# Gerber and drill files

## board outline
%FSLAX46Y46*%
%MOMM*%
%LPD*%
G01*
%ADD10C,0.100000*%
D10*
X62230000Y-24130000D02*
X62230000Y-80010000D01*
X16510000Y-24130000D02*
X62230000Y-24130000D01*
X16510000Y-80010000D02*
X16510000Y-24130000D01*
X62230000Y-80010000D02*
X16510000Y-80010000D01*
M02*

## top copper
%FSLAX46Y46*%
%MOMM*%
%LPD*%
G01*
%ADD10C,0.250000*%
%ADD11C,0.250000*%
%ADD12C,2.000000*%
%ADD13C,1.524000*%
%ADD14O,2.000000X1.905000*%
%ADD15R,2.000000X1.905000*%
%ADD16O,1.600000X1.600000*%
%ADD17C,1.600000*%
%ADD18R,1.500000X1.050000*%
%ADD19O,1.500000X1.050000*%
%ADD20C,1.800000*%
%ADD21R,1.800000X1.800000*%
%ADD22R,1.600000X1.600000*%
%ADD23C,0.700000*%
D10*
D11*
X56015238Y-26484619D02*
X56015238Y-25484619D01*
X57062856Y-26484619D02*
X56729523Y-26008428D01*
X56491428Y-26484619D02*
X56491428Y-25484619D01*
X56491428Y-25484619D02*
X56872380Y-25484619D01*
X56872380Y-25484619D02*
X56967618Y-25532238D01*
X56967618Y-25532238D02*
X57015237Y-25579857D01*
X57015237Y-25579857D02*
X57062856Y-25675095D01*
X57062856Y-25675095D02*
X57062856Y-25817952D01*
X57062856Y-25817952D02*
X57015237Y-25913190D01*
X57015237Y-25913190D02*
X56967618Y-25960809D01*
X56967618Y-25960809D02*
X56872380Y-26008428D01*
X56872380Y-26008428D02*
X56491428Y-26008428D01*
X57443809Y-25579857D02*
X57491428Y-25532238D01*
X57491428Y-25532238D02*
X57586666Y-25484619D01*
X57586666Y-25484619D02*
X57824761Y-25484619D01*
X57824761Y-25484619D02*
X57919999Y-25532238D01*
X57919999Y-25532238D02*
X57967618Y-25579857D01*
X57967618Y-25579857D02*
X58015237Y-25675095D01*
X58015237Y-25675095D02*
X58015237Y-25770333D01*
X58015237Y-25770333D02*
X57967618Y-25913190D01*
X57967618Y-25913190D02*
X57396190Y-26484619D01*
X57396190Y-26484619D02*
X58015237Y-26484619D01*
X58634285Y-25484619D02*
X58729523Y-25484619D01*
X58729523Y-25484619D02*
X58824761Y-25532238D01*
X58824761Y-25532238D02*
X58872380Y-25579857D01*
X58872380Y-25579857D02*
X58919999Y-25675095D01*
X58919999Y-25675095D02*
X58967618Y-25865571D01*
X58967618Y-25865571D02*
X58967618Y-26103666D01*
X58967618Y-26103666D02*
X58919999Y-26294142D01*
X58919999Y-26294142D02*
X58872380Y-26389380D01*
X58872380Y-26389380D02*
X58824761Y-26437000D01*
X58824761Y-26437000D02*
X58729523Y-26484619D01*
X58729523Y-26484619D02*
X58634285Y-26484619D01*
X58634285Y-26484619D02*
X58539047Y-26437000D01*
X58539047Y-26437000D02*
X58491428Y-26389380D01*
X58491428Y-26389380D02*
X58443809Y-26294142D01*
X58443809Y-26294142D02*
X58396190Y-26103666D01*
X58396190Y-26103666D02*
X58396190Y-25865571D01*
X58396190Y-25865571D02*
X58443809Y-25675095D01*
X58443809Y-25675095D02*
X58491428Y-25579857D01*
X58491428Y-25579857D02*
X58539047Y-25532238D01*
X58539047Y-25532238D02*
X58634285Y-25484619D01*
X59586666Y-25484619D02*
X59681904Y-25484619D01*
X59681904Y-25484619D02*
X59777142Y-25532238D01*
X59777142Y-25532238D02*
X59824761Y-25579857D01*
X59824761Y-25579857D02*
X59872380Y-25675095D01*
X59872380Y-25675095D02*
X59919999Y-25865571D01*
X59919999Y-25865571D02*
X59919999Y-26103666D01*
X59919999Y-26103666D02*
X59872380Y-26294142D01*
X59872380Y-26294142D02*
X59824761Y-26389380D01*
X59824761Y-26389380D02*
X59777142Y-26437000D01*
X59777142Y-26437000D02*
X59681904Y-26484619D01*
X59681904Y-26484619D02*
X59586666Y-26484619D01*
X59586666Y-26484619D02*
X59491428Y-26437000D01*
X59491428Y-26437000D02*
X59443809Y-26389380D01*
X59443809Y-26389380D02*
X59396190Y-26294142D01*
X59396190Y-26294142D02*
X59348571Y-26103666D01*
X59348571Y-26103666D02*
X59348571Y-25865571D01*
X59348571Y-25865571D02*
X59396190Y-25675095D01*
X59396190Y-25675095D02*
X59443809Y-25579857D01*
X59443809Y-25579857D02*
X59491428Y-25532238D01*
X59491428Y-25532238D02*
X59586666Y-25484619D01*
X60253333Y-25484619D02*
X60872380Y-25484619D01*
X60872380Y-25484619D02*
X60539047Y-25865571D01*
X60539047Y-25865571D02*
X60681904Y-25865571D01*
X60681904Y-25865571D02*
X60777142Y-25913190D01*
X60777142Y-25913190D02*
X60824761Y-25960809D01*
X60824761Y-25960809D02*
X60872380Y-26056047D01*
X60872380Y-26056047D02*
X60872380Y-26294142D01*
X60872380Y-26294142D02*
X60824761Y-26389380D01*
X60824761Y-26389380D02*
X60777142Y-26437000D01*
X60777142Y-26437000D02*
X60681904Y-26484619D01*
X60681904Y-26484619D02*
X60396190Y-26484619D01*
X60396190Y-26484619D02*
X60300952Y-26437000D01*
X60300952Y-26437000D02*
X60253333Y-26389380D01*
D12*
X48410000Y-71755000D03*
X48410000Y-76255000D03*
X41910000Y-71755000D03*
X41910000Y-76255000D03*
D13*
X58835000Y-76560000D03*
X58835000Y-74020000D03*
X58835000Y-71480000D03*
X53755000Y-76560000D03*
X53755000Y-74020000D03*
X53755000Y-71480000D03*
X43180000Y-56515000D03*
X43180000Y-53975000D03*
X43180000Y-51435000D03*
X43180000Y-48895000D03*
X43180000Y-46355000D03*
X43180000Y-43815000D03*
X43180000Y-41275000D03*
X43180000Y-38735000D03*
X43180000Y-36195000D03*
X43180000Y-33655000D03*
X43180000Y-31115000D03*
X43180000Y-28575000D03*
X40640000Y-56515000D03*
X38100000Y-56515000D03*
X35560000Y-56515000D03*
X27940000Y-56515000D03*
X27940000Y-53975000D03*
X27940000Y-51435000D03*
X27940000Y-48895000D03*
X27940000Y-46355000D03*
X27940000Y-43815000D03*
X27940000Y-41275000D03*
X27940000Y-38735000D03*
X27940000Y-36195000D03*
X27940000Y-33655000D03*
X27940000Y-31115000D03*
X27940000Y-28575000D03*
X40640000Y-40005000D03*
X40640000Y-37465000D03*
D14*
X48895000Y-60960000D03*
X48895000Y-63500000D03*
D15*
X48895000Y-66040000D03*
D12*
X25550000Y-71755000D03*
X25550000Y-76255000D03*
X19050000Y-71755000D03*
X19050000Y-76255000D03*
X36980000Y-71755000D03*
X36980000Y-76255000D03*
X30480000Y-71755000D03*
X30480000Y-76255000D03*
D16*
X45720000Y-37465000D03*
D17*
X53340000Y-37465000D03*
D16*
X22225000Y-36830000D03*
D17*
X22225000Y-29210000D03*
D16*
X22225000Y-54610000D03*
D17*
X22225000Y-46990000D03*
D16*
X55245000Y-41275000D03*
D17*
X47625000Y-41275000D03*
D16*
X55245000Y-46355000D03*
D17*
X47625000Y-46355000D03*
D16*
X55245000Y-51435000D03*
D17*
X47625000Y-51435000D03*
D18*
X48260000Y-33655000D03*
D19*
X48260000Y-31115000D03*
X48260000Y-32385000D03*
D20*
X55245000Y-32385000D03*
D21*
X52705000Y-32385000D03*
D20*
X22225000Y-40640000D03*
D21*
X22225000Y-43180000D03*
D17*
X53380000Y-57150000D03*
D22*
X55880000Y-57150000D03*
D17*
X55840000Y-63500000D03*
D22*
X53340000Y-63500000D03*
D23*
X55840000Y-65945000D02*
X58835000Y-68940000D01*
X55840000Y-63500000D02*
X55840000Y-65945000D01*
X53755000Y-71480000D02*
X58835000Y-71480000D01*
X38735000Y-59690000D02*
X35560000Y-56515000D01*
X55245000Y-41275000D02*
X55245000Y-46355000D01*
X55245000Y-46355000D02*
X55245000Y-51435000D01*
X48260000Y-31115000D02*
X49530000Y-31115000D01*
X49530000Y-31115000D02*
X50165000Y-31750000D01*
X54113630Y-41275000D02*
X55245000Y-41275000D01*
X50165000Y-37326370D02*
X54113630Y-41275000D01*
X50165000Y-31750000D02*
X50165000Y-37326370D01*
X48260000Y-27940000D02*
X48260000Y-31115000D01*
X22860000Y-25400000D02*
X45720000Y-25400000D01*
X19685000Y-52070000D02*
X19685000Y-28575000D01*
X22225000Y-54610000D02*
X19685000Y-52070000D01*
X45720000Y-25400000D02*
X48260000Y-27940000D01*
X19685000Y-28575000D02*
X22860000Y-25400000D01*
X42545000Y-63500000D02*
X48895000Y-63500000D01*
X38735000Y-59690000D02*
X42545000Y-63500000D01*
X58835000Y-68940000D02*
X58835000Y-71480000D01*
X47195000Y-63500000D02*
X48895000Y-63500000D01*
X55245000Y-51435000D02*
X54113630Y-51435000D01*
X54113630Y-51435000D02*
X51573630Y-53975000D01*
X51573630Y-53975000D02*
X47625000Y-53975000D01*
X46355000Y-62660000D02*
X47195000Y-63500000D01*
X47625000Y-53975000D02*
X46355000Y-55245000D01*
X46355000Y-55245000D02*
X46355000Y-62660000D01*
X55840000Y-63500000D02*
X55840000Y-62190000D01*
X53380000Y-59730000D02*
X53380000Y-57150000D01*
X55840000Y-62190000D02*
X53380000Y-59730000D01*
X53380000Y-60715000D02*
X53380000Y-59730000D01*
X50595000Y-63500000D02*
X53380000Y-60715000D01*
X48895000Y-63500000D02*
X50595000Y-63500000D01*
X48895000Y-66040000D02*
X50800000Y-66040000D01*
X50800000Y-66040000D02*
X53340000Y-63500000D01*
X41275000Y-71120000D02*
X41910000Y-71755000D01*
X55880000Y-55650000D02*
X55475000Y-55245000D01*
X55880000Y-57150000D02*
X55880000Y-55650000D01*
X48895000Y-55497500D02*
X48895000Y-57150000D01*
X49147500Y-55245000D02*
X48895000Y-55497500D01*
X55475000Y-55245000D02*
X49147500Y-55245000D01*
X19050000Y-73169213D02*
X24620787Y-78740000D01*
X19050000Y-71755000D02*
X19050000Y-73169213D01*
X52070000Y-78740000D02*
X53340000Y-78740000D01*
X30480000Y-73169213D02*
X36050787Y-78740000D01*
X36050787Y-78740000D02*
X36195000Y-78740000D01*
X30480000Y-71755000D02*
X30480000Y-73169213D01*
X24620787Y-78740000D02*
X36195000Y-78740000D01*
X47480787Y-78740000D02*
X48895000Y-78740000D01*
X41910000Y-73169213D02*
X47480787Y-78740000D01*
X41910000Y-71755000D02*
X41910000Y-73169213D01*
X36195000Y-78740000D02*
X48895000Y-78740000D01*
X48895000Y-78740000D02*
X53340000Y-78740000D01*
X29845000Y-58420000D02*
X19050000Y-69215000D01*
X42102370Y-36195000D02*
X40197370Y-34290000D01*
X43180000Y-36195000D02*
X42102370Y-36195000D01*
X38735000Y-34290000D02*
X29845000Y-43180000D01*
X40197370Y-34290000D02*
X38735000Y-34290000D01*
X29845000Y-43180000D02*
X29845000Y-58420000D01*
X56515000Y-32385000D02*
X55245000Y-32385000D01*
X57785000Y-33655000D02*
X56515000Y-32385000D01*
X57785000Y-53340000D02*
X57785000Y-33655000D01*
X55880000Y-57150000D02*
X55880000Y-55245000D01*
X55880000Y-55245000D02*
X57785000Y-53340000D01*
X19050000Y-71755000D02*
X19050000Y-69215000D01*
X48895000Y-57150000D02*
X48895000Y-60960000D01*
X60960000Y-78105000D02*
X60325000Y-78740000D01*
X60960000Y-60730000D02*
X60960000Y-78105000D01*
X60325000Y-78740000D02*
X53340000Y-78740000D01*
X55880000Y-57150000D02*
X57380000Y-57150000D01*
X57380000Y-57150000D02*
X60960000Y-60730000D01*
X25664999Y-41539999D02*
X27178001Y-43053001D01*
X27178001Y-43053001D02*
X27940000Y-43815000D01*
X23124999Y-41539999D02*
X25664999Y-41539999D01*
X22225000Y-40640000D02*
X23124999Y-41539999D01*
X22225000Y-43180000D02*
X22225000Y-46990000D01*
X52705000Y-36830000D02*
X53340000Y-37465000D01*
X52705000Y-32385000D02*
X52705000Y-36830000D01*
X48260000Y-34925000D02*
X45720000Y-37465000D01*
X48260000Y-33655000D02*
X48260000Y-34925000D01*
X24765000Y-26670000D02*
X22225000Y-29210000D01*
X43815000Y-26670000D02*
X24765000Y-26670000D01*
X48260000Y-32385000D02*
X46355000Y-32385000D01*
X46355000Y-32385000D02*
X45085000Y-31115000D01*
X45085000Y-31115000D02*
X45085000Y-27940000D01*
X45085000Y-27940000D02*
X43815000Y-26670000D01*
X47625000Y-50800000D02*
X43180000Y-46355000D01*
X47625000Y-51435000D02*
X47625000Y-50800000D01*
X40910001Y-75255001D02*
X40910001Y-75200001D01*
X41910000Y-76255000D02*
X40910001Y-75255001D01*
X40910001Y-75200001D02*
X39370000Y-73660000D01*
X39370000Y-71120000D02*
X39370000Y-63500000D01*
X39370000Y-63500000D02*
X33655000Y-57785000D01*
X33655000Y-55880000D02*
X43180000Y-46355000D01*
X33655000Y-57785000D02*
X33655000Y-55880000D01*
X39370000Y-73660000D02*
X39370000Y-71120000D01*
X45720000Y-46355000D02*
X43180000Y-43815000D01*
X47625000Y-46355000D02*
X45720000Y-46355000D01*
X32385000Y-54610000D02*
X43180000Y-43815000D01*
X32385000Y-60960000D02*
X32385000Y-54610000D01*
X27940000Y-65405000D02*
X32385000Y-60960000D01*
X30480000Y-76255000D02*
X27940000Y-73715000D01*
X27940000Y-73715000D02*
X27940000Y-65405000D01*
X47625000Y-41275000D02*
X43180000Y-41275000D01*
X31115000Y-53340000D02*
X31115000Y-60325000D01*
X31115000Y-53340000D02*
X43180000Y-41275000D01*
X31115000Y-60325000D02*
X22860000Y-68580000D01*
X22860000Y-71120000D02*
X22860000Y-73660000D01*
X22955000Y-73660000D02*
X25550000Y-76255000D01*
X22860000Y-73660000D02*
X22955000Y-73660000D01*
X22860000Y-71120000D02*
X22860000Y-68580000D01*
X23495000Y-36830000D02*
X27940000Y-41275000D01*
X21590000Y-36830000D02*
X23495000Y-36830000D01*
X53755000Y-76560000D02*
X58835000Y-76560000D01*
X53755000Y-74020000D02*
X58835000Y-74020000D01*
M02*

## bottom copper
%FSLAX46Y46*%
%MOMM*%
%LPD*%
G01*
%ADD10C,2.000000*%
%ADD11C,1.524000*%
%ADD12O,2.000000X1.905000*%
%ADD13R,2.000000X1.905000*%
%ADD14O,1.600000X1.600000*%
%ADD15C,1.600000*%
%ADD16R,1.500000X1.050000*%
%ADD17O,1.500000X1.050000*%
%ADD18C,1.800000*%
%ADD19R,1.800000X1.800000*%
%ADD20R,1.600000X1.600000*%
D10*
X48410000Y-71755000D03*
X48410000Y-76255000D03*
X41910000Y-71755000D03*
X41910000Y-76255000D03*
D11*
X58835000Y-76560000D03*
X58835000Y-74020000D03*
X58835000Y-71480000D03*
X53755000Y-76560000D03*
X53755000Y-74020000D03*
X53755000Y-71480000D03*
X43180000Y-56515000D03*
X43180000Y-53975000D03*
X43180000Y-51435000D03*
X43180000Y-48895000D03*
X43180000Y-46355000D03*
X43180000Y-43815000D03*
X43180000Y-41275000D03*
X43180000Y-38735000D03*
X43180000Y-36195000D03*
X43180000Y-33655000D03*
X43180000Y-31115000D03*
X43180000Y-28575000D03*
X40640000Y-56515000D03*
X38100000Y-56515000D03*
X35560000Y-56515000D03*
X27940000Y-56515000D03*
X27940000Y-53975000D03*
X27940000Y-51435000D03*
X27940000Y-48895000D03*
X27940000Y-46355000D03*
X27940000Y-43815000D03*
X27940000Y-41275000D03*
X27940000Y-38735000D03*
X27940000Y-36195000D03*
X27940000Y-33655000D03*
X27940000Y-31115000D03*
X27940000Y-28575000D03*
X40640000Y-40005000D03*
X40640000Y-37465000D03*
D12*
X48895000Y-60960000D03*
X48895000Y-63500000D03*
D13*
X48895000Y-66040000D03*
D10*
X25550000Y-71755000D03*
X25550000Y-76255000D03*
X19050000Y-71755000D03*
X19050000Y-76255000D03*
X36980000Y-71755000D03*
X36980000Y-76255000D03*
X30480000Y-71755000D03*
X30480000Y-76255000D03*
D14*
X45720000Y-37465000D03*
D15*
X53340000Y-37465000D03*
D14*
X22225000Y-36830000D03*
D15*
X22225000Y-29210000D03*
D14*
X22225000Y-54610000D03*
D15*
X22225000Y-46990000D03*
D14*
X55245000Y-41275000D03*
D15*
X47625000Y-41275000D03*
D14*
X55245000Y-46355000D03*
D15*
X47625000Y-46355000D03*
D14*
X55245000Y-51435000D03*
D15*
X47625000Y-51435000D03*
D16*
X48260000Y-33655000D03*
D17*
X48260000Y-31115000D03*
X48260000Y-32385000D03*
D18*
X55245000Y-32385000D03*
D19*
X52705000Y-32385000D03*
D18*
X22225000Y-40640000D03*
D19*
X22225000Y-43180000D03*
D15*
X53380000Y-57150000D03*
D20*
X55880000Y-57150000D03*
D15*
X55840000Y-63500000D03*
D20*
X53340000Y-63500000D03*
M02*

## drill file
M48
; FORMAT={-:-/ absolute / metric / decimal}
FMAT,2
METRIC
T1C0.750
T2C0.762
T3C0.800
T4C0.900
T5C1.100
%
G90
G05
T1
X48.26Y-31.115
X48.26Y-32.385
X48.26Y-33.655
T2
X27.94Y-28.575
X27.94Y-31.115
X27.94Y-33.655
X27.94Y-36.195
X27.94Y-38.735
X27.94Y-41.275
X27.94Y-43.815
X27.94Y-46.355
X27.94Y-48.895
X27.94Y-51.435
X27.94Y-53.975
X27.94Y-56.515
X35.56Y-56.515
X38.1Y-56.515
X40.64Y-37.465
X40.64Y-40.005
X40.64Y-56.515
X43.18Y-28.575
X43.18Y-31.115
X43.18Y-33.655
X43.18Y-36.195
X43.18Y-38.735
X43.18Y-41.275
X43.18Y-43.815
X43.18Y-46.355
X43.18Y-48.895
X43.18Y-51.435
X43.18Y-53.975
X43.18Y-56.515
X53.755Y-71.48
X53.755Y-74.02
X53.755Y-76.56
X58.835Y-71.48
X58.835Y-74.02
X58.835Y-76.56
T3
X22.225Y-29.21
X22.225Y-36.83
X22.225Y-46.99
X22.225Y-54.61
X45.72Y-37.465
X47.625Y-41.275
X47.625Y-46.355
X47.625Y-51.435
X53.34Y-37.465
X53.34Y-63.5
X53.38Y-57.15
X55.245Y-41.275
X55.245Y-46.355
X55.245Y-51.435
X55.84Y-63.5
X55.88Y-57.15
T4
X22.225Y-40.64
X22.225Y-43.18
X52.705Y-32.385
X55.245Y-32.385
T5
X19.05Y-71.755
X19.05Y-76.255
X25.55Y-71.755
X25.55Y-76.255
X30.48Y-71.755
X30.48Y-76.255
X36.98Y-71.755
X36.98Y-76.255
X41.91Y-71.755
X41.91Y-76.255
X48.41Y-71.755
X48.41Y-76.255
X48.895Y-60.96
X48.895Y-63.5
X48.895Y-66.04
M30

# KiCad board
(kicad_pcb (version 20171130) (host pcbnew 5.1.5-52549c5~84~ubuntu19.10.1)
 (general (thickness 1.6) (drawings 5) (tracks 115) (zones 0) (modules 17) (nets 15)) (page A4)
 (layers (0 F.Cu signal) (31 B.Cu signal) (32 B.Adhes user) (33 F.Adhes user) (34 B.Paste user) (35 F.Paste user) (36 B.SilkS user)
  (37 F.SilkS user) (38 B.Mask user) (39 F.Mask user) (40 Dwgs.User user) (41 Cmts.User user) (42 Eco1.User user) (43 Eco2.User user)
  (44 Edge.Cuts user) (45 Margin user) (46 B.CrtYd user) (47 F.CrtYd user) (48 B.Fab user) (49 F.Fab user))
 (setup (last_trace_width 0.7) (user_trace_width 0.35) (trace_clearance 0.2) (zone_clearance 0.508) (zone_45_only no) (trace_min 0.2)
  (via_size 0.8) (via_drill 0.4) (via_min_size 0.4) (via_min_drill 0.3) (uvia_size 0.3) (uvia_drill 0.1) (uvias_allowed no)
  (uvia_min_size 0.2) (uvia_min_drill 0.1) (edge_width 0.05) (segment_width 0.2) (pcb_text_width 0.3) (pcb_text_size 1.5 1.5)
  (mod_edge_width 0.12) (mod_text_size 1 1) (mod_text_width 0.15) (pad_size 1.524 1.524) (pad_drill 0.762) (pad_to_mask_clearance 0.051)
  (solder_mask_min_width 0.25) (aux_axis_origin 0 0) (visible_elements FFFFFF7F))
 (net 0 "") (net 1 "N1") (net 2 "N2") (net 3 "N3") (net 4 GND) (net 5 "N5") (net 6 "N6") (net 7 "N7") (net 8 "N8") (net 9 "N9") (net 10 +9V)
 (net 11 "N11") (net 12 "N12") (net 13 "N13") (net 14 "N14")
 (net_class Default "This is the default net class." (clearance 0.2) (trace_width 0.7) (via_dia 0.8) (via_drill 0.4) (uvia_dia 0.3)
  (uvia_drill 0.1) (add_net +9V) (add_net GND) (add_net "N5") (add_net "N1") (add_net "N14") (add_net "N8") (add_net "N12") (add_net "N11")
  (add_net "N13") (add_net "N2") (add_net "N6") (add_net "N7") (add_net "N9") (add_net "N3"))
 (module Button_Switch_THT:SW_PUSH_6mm (layer F.Cu) (at 41.91 71.755)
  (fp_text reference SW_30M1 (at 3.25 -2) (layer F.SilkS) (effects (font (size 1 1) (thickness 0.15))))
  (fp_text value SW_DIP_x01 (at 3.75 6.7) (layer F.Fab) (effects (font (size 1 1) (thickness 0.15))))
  (pad 1 thru_hole circle (at 6.5 0 90) (size 2 2) (drill 1.1) (layers *.Cu *.Mask) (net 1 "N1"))
  (pad 2 thru_hole circle (at 6.5 4.5 90) (size 2 2) (drill 1.1) (layers *.Cu *.Mask) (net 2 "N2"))
  (pad 1 thru_hole circle (at 0 0 90) (size 2 2) (drill 1.1) (layers *.Cu *.Mask) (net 1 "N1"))
  (pad 2 thru_hole circle (at 0 4.5 90) (size 2 2) (drill 1.1) (layers *.Cu *.Mask) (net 2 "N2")))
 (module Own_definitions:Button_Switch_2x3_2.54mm (layer F.Cu) (at 51.215 68.94)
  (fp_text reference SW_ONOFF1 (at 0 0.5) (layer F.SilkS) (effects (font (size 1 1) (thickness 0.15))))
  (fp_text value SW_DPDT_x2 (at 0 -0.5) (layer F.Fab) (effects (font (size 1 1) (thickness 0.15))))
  (pad 3 thru_hole circle (at 7.62 7.62) (size 1.524 1.524) (drill 0.762) (layers *.Cu *.Mask) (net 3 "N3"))
  (pad 2 thru_hole circle (at 7.62 5.08) (size 1.524 1.524) (drill 0.762) (layers *.Cu *.Mask) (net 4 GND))
  (pad 1 thru_hole circle (at 7.62 2.54) (size 1.524 1.524) (drill 0.762) (layers *.Cu *.Mask) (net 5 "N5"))
  (pad 3 thru_hole circle (at 2.54 7.62) (size 1.524 1.524) (drill 0.762) (layers *.Cu *.Mask) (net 3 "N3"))
  (pad 2 thru_hole circle (at 2.54 5.08) (size 1.524 1.524) (drill 0.762) (layers *.Cu *.Mask) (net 4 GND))
  (pad 1 thru_hole circle (at 2.54 2.54) (size 1.524 1.524) (drill 0.762) (layers *.Cu *.Mask) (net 5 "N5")))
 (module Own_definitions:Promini (layer F.Cu) (at 26.67 23.495)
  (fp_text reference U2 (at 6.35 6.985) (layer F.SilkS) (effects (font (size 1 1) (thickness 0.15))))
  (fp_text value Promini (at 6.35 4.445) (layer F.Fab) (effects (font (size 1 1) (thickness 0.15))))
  (pad 16 thru_hole circle (at 16.51 33.02) (size 1.524 1.524) (drill 0.762) (layers *.Cu *.Mask))
  (pad 17 thru_hole circle (at 16.51 30.48) (size 1.524 1.524) (drill 0.762) (layers *.Cu *.Mask))
  (pad 18 thru_hole circle (at 16.51 27.94) (size 1.524 1.524) (drill 0.762) (layers *.Cu *.Mask))
  (pad 19 thru_hole circle (at 16.51 25.4) (size 1.524 1.524) (drill 0.762) (layers *.Cu *.Mask))
  (pad 20 thru_hole circle (at 16.51 22.86) (size 1.524 1.524) (drill 0.762) (layers *.Cu *.Mask) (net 2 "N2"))
  (pad 21 thru_hole circle (at 16.51 20.32) (size 1.524 1.524) (drill 0.762) (layers *.Cu *.Mask) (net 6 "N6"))
  (pad 22 thru_hole circle (at 16.51 17.78) (size 1.524 1.524) (drill 0.762) (layers *.Cu *.Mask) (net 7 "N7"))
  (pad 23 thru_hole circle (at 16.51 15.24) (size 1.524 1.524) (drill 0.762) (layers *.Cu *.Mask))
  (pad 24 thru_hole circle (at 16.51 12.7) (size 1.524 1.524) (drill 0.762) (layers *.Cu *.Mask) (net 1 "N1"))
  (pad 25 thru_hole circle (at 16.51 10.16) (size 1.524 1.524) (drill 0.762) (layers *.Cu *.Mask))
  (pad 26 thru_hole circle (at 16.51 7.62) (size 1.524 1.524) (drill 0.762) (layers *.Cu *.Mask))
  (pad 27 thru_hole circle (at 16.51 5.08) (size 1.524 1.524) (drill 0.762) (layers *.Cu *.Mask))
  (pad 15 thru_hole circle (at 13.97 33.02) (size 1.524 1.524) (drill 0.762) (layers *.Cu *.Mask))
  (pad 14 thru_hole circle (at 11.43 33.02) (size 1.524 1.524) (drill 0.762) (layers *.Cu *.Mask))
  (pad 13 thru_hole circle (at 8.89 33.02) (size 1.524 1.524) (drill 0.762) (layers *.Cu *.Mask) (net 5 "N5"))
  (pad 12 thru_hole circle (at 1.27 33.02) (size 1.524 1.524) (drill 0.762) (layers *.Cu *.Mask))
  (pad 11 thru_hole circle (at 1.27 30.48) (size 1.524 1.524) (drill 0.762) (layers *.Cu *.Mask))
  (pad 10 thru_hole circle (at 1.27 27.94) (size 1.524 1.524) (drill 0.762) (layers *.Cu *.Mask))
  (pad 9 thru_hole circle (at 1.27 25.4) (size 1.524 1.524) (drill 0.762) (layers *.Cu *.Mask))
  (pad 8 thru_hole circle (at 1.27 22.86) (size 1.524 1.524) (drill 0.762) (layers *.Cu *.Mask))
  (pad 7 thru_hole circle (at 1.27 20.32) (size 1.524 1.524) (drill 0.762) (layers *.Cu *.Mask) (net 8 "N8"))
  (pad 6 thru_hole circle (at 1.27 17.78) (size 1.524 1.524) (drill 0.762) (layers *.Cu *.Mask) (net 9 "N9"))
  (pad 5 thru_hole circle (at 1.27 15.24) (size 1.524 1.524) (drill 0.762) (layers *.Cu *.Mask))
  (pad 4 thru_hole circle (at 1.27 12.7) (size 1.524 1.524) (drill 0.762) (layers *.Cu *.Mask))
  (pad 3 thru_hole circle (at 1.27 10.16) (size 1.524 1.524) (drill 0.762) (layers *.Cu *.Mask))
  (pad 2 thru_hole circle (at 1.27 7.62) (size 1.524 1.524) (drill 0.762) (layers *.Cu *.Mask))
  (pad 1 thru_hole circle (at 1.27 5.08) (size 1.524 1.524) (drill 0.762) (layers *.Cu *.Mask))
  (pad 28 thru_hole circle (at 13.97 16.51) (size 1.524 1.524) (drill 0.762) (layers *.Cu *.Mask))
  (pad 29 thru_hole circle (at 13.97 13.97) (size 1.524 1.524) (drill 0.762) (layers *.Cu *.Mask)))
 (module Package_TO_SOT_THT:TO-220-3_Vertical (layer F.Cu) (at 48.895 66.04 90)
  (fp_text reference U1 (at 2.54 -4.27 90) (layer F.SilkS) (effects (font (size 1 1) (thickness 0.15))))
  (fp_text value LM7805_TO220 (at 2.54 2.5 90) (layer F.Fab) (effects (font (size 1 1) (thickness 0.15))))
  (pad 3 thru_hole oval (at 5.08 0 90) (size 1.905 2) (drill 1.1) (layers *.Cu *.Mask) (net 1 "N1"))
  (pad 2 thru_hole oval (at 2.54 0 90) (size 1.905 2) (drill 1.1) (layers *.Cu *.Mask) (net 5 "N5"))
  (pad 1 thru_hole rect (at 0 0 90) (size 1.905 2) (drill 1.1) (layers *.Cu *.Mask) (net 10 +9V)))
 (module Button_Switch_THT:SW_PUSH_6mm (layer F.Cu) (at 19.05 71.755)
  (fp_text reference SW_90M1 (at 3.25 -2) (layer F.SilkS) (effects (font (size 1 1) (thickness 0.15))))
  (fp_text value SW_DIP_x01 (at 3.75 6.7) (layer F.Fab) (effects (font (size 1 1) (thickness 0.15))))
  (pad 1 thru_hole circle (at 6.5 0 90) (size 2 2) (drill 1.1) (layers *.Cu *.Mask) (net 1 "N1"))
  (pad 2 thru_hole circle (at 6.5 4.5 90) (size 2 2) (drill 1.1) (layers *.Cu *.Mask) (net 7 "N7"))
  (pad 1 thru_hole circle (at 0 0 90) (size 2 2) (drill 1.1) (layers *.Cu *.Mask) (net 1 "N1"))
  (pad 2 thru_hole circle (at 0 4.5 90) (size 2 2) (drill 1.1) (layers *.Cu *.Mask) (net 7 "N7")))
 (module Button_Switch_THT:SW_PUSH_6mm (layer F.Cu) (at 30.48 71.755)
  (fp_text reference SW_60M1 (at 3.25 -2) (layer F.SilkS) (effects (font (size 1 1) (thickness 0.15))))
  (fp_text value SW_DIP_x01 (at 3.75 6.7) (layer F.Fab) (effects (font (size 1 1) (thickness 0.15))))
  (pad 1 thru_hole circle (at 6.5 0 90) (size 2 2) (drill 1.1) (layers *.Cu *.Mask) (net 1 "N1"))
  (pad 2 thru_hole circle (at 6.5 4.5 90) (size 2 2) (drill 1.1) (layers *.Cu *.Mask) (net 6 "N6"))
  (pad 1 thru_hole circle (at 0 0 90) (size 2 2) (drill 1.1) (layers *.Cu *.Mask) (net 1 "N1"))
  (pad 2 thru_hole circle (at 0 4.5 90) (size 2 2) (drill 1.1) (layers *.Cu *.Mask) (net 6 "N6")))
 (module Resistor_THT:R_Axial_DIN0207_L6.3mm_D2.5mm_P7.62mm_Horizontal (layer F.Cu) (at 53.34 37.465 180)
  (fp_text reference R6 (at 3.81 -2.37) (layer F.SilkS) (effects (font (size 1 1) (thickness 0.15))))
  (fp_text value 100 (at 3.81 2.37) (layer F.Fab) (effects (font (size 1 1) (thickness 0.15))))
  (pad 2 thru_hole oval (at 7.62 0 180) (size 1.6 1.6) (drill 0.8) (layers *.Cu *.Mask) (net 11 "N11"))
  (pad 1 thru_hole circle (at 0 0 180) (size 1.6 1.6) (drill 0.8) (layers *.Cu *.Mask) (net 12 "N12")))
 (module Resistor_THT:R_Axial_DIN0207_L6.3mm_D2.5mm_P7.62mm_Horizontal (layer F.Cu) (at 22.225 29.21 270)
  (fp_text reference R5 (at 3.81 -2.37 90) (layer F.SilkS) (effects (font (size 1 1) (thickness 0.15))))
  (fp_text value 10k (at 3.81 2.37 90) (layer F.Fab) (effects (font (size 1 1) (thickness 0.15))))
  (pad 2 thru_hole oval (at 7.62 0 270) (size 1.6 1.6) (drill 0.8) (layers *.Cu *.Mask) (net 9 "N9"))
  (pad 1 thru_hole circle (at 0 0 270) (size 1.6 1.6) (drill 0.8) (layers *.Cu *.Mask) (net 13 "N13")))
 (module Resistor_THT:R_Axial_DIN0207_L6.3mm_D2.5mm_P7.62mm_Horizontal (layer F.Cu) (at 22.225 46.99 270)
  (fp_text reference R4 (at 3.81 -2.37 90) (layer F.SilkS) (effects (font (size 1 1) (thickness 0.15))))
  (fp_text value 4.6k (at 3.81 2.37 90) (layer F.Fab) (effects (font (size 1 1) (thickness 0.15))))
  (pad 2 thru_hole oval (at 7.62 0 270) (size 1.6 1.6) (drill 0.8) (layers *.Cu *.Mask) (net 5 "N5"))
  (pad 1 thru_hole circle (at 0 0 270) (size 1.6 1.6) (drill 0.8) (layers *.Cu *.Mask) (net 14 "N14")))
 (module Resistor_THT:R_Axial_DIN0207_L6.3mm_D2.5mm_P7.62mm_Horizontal (layer F.Cu) (at 47.625 41.275)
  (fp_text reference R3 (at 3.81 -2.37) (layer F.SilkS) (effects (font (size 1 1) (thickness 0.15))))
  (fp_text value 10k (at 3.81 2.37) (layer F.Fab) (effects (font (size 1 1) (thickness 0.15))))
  (pad 2 thru_hole oval (at 7.62 0) (size 1.6 1.6) (drill 0.8) (layers *.Cu *.Mask) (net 5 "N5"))
  (pad 1 thru_hole circle (at 0 0) (size 1.6 1.6) (drill 0.8) (layers *.Cu *.Mask) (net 7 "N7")))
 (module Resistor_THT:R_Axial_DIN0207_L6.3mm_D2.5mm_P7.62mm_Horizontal (layer F.Cu) (at 47.625 46.355)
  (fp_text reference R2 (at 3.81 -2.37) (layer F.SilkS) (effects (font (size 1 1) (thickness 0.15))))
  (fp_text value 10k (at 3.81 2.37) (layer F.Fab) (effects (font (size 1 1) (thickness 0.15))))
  (pad 2 thru_hole oval (at 7.62 0) (size 1.6 1.6) (drill 0.8) (layers *.Cu *.Mask) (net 5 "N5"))
  (pad 1 thru_hole circle (at 0 0) (size 1.6 1.6) (drill 0.8) (layers *.Cu *.Mask) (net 6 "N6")))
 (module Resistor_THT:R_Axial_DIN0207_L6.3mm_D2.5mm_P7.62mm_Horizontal (layer F.Cu) (at 47.625 51.435)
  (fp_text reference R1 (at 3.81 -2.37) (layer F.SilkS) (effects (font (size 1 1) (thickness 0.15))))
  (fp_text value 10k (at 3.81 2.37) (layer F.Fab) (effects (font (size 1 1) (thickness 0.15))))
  (pad 2 thru_hole oval (at 7.62 0) (size 1.6 1.6) (drill 0.8) (layers *.Cu *.Mask) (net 5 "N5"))
  (pad 1 thru_hole circle (at 0 0) (size 1.6 1.6) (drill 0.8) (layers *.Cu *.Mask) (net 2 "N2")))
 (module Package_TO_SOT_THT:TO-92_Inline (layer F.Cu) (at 48.26 33.655 90)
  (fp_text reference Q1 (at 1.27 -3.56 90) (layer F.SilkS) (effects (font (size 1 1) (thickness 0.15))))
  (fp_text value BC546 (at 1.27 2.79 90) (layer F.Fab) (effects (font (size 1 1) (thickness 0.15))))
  (pad 1 thru_hole rect (at 0 0 90) (size 1.05 1.5) (drill 0.75) (layers *.Cu *.Mask) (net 11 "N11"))
  (pad 3 thru_hole oval (at 2.54 0 90) (size 1.05 1.5) (drill 0.75) (layers *.Cu *.Mask) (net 5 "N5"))
  (pad 2 thru_hole oval (at 1.27 0 90) (size 1.05 1.5) (drill 0.75) (layers *.Cu *.Mask) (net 13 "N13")))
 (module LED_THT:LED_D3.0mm (layer F.Cu) (at 52.705 32.385)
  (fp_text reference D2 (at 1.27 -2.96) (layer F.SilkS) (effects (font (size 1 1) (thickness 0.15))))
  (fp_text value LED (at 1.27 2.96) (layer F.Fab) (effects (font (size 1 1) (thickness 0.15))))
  (pad 2 thru_hole circle (at 2.54 0) (size 1.8 1.8) (drill 0.9) (layers *.Cu *.Mask) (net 1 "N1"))
  (pad 1 thru_hole rect (at 0 0) (size 1.8 1.8) (drill 0.9) (layers *.Cu *.Mask) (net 12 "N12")))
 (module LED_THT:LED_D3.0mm (layer F.Cu) (at 22.225 43.18 90)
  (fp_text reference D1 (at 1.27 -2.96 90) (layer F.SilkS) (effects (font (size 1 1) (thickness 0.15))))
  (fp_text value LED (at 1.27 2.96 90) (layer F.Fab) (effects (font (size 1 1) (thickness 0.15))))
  (pad 2 thru_hole circle (at 2.54 0 90) (size 1.8 1.8) (drill 0.9) (layers *.Cu *.Mask) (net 8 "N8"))
  (pad 1 thru_hole rect (at 0 0 90) (size 1.8 1.8) (drill 0.9) (layers *.Cu *.Mask) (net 14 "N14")))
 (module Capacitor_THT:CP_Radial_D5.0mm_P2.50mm (layer F.Cu) (at 55.88 57.15 180)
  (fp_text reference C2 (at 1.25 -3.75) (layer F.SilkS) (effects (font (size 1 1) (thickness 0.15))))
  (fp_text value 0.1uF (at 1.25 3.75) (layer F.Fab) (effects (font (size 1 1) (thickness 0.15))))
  (pad 2 thru_hole circle (at 2.5 0 180) (size 1.6 1.6) (drill 0.8) (layers *.Cu *.Mask) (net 5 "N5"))
  (pad 1 thru_hole rect (at 0 0 180) (size 1.6 1.6) (drill 0.8) (layers *.Cu *.Mask) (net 1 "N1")))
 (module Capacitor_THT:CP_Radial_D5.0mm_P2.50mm (layer F.Cu) (at 53.34 63.5)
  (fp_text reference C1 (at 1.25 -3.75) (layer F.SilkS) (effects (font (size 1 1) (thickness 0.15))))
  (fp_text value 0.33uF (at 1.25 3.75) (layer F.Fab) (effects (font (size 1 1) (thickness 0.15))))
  (pad 2 thru_hole circle (at 2.5 0) (size 1.6 1.6) (drill 0.8) (layers *.Cu *.Mask) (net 5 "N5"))
  (pad 1 thru_hole rect (at 0 0) (size 1.6 1.6) (drill 0.8) (layers *.Cu *.Mask) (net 10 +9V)))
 (gr_line (start 62.23 24.13) (end 62.23 80.01) (layer Edge.Cuts) (width 0.1))
 (gr_line (start 16.51 24.13) (end 62.23 24.13) (layer Edge.Cuts) (width 0.1))
 (gr_line (start 16.51 80.01) (end 16.51 24.13) (layer Edge.Cuts) (width 0.1))
 (gr_line (start 62.23 80.01) (end 16.51 80.01) (layer Edge.Cuts) (width 0.1))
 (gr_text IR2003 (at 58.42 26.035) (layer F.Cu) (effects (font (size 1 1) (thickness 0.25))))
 (segment (start 55.84 65.945) (end 58.835 68.94) (width 0.7) (layer F.Cu) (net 5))
 (segment (start 55.84 63.5) (end 55.84 65.945) (width 0.7) (layer F.Cu) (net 5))
 (segment (start 53.755 71.48) (end 58.835 71.48) (width 0.7) (layer F.Cu) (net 5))
 (segment (start 38.735 59.69) (end 35.56 56.515) (width 0.7) (layer F.Cu) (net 5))
 (segment (start 55.245 41.275) (end 55.245 46.355) (width 0.7) (layer F.Cu) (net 5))
 (segment (start 55.245 46.355) (end 55.245 51.435) (width 0.7) (layer F.Cu) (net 5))
 (segment (start 48.26 31.115) (end 49.53 31.115) (width 0.7) (layer F.Cu) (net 5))
 (segment (start 49.53 31.115) (end 50.165 31.75) (width 0.7) (layer F.Cu) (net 5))
 (segment (start 54.11363 41.275) (end 55.245 41.275) (width 0.7) (layer F.Cu) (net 5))
 (segment (start 50.165 37.32637) (end 54.11363 41.275) (width 0.7) (layer F.Cu) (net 5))
 (segment (start 50.165 31.75) (end 50.165 37.32637) (width 0.7) (layer F.Cu) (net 5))
 (segment (start 48.26 27.94) (end 48.26 31.115) (width 0.7) (layer F.Cu) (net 5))
 (segment (start 22.86 25.4) (end 45.72 25.4) (width 0.7) (layer F.Cu) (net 5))
 (segment (start 19.685 52.07) (end 19.685 28.575) (width 0.7) (layer F.Cu) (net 5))
 (segment (start 22.225 54.61) (end 19.685 52.07) (width 0.7) (layer F.Cu) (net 5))
 (segment (start 45.72 25.4) (end 48.26 27.94) (width 0.7) (layer F.Cu) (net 5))
 (segment (start 19.685 28.575) (end 22.86 25.4) (width 0.7) (layer F.Cu) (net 5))
 (segment (start 42.545 63.5) (end 48.895 63.5) (width 0.7) (layer F.Cu) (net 5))
 (segment (start 38.735 59.69) (end 42.545 63.5) (width 0.7) (layer F.Cu) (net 5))
 (segment (start 58.835 68.94) (end 58.835 71.48) (width 0.7) (layer F.Cu) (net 5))
 (segment (start 47.195 63.5) (end 48.895 63.5) (width 0.7) (layer F.Cu) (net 5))
 (segment (start 55.245 51.435) (end 54.11363 51.435) (width 0.7) (layer F.Cu) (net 5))
 (segment (start 54.11363 51.435) (end 51.57363 53.975) (width 0.7) (layer F.Cu) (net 5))
 (segment (start 51.57363 53.975) (end 47.625 53.975) (width 0.7) (layer F.Cu) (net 5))
 (segment (start 46.355 62.66) (end 47.195 63.5) (width 0.7) (layer F.Cu) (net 5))
 (segment (start 47.625 53.975) (end 46.355 55.245) (width 0.7) (layer F.Cu) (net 5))
 (segment (start 46.355 55.245) (end 46.355 62.66) (width 0.7) (layer F.Cu) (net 5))
 (segment (start 55.84 63.5) (end 55.84 62.19) (width 0.7) (layer F.Cu) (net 5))
 (segment (start 53.38 59.73) (end 53.38 57.15) (width 0.7) (layer F.Cu) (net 5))
 (segment (start 55.84 62.19) (end 53.38 59.73) (width 0.7) (layer F.Cu) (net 5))
 (segment (start 53.38 60.715) (end 53.38 59.73) (width 0.7) (layer F.Cu) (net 5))
 (segment (start 50.595 63.5) (end 53.38 60.715) (width 0.7) (layer F.Cu) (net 5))
 (segment (start 48.895 63.5) (end 50.595 63.5) (width 0.7) (layer F.Cu) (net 5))
 (segment (start 48.895 66.04) (end 50.8 66.04) (width 0.7) (layer F.Cu) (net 10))
 (segment (start 50.8 66.04) (end 53.34 63.5) (width 0.7) (layer F.Cu) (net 10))
 (segment (start 41.275 71.12) (end 41.91 71.755) (width 0.7) (layer F.Cu) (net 1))
 (segment (start 55.88 55.65) (end 55.475 55.245) (width 0.7) (layer F.Cu) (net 1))
 (segment (start 55.88 57.15) (end 55.88 55.65) (width 0.7) (layer F.Cu) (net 1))
 (segment (start 48.895 55.4975) (end 48.895 57.15) (width 0.7) (layer F.Cu) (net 1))
 (segment (start 49.1475 55.245) (end 48.895 55.4975) (width 0.7) (layer F.Cu) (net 1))
 (segment (start 55.475 55.245) (end 49.1475 55.245) (width 0.7) (layer F.Cu) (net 1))
 (segment (start 19.05 73.169213) (end 24.620787 78.74) (width 0.7) (layer F.Cu) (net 1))
 (segment (start 19.05 71.755) (end 19.05 73.169213) (width 0.7) (layer F.Cu) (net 1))
 (segment (start 52.07 78.74) (end 53.34 78.74) (width 0.7) (layer F.Cu) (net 1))
 (segment (start 30.48 73.169213) (end 36.050787 78.74) (width 0.7) (layer F.Cu) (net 1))
 (segment (start 36.050787 78.74) (end 36.195 78.74) (width 0.7) (layer F.Cu) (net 1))
 (segment (start 30.48 71.755) (end 30.48 73.169213) (width 0.7) (layer F.Cu) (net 1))
 (segment (start 24.620787 78.74) (end 36.195 78.74) (width 0.7) (layer F.Cu) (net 1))
 (segment (start 47.480787 78.74) (end 48.895 78.74) (width 0.7) (layer F.Cu) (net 1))
 (segment (start 41.91 73.169213) (end 47.480787 78.74) (width 0.7) (layer F.Cu) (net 1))
 (segment (start 41.91 71.755) (end 41.91 73.169213) (width 0.7) (layer F.Cu) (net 1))
 (segment (start 36.195 78.74) (end 48.895 78.74) (width 0.7) (layer F.Cu) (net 1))
 (segment (start 48.895 78.74) (end 53.34 78.74) (width 0.7) (layer F.Cu) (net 1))
 (segment (start 29.845 58.42) (end 19.05 69.215) (width 0.7) (layer F.Cu) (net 1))
 (segment (start 42.10237 36.195) (end 40.19737 34.29) (width 0.7) (layer F.Cu) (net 1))
 (segment (start 43.18 36.195) (end 42.10237 36.195) (width 0.7) (layer F.Cu) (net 1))
 (segment (start 38.735 34.29) (end 29.845 43.18) (width 0.7) (layer F.Cu) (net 1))
 (segment (start 40.19737 34.29) (end 38.735 34.29) (width 0.7) (layer F.Cu) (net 1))
 (segment (start 29.845 43.18) (end 29.845 58.42) (width 0.7) (layer F.Cu) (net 1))
 (segment (start 56.515 32.385) (end 55.245 32.385) (width 0.7) (layer F.Cu) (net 1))
 (segment (start 57.785 33.655) (end 56.515 32.385) (width 0.7) (layer F.Cu) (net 1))
 (segment (start 57.785 53.34) (end 57.785 33.655) (width 0.7) (layer F.Cu) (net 1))
 (segment (start 55.88 57.15) (end 55.88 55.245) (width 0.7) (layer F.Cu) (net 1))
 (segment (start 55.88 55.245) (end 57.785 53.34) (width 0.7) (layer F.Cu) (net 1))
 (segment (start 19.05 71.755) (end 19.05 69.215) (width 0.7) (layer F.Cu) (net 1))
 (segment (start 48.895 57.15) (end 48.895 60.96) (width 0.7) (layer F.Cu) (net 1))
 (segment (start 60.96 78.105) (end 60.325 78.74) (width 0.7) (layer F.Cu) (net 1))
 (segment (start 60.96 60.73) (end 60.96 78.105) (width 0.7) (layer F.Cu) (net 1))
 (segment (start 60.325 78.74) (end 53.34 78.74) (width 0.7) (layer F.Cu) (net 1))
 (segment (start 55.88 57.15) (end 57.38 57.15) (width 0.7) (layer F.Cu) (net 1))
 (segment (start 57.38 57.15) (end 60.96 60.73) (width 0.7) (layer F.Cu) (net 1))
 (segment (start 25.664999 41.539999) (end 27.178001 43.053001) (width 0.7) (layer F.Cu) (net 8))
 (segment (start 27.178001 43.053001) (end 27.94 43.815) (width 0.7) (layer F.Cu) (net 8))
 (segment (start 23.124999 41.539999) (end 25.664999 41.539999) (width 0.7) (layer F.Cu) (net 8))
 (segment (start 22.225 40.64) (end 23.124999 41.539999) (width 0.7) (layer F.Cu) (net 8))
 (segment (start 22.225 43.18) (end 22.225 46.99) (width 0.7) (layer F.Cu) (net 14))
 (segment (start 52.705 36.83) (end 53.34 37.465) (width 0.7) (layer F.Cu) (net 12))
 (segment (start 52.705 32.385) (end 52.705 36.83) (width 0.7) (layer F.Cu) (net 12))
 (segment (start 48.26 34.925) (end 45.72 37.465) (width 0.7) (layer F.Cu) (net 11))
 (segment (start 48.26 33.655) (end 48.26 34.925) (width 0.7) (layer F.Cu) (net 11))
 (segment (start 24.765 26.67) (end 22.225 29.21) (width 0.7) (layer F.Cu) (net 13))
 (segment (start 43.815 26.67) (end 24.765 26.67) (width 0.7) (layer F.Cu) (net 13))
 (segment (start 48.26 32.385) (end 46.355 32.385) (width 0.7) (layer F.Cu) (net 13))
 (segment (start 46.355 32.385) (end 45.085 31.115) (width 0.7) (layer F.Cu) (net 13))
 (segment (start 45.085 31.115) (end 45.085 27.94) (width 0.7) (layer F.Cu) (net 13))
 (segment (start 45.085 27.94) (end 43.815 26.67) (width 0.7) (layer F.Cu) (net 13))
 (segment (start 47.625 50.8) (end 43.18 46.355) (width 0.7) (layer F.Cu) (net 2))
 (segment (start 47.625 51.435) (end 47.625 50.8) (width 0.7) (layer F.Cu) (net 2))
 (segment (start 40.910001 75.255001) (end 40.910001 75.200001) (width 0.7) (layer F.Cu) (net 2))
 (segment (start 41.91 76.255) (end 40.910001 75.255001) (width 0.7) (layer F.Cu) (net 2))
 (segment (start 40.910001 75.200001) (end 39.37 73.66) (width 0.7) (layer F.Cu) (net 2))
 (segment (start 39.37 71.12) (end 39.37 63.5) (width 0.7) (layer F.Cu) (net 2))
 (segment (start 39.37 63.5) (end 33.655 57.785) (width 0.7) (layer F.Cu) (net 2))
 (segment (start 33.655 55.88) (end 43.18 46.355) (width 0.7) (layer F.Cu) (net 2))
 (segment (start 33.655 57.785) (end 33.655 55.88) (width 0.7) (layer F.Cu) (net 2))
 (segment (start 39.37 73.66) (end 39.37 71.12) (width 0.7) (layer F.Cu) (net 2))
 (segment (start 45.72 46.355) (end 43.18 43.815) (width 0.7) (layer F.Cu) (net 6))
 (segment (start 47.625 46.355) (end 45.72 46.355) (width 0.7) (layer F.Cu) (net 6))
 (segment (start 32.385 54.61) (end 43.18 43.815) (width 0.7) (layer F.Cu) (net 6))
 (segment (start 32.385 60.96) (end 32.385 54.61) (width 0.7) (layer F.Cu) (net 6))
 (segment (start 27.94 65.405) (end 32.385 60.96) (width 0.7) (layer F.Cu) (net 6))
 (segment (start 30.48 76.255) (end 27.94 73.715) (width 0.7) (layer F.Cu) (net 6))
 (segment (start 27.94 73.715) (end 27.94 65.405) (width 0.7) (layer F.Cu) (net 6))
 (segment (start 47.625 41.275) (end 43.18 41.275) (width 0.7) (layer F.Cu) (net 7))
 (segment (start 31.115 53.34) (end 31.115 60.325) (width 0.7) (layer F.Cu) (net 7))
 (segment (start 31.115 53.34) (end 43.18 41.275) (width 0.7) (layer F.Cu) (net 7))
 (segment (start 31.115 60.325) (end 22.86 68.58) (width 0.7) (layer F.Cu) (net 7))
 (segment (start 22.86 71.12) (end 22.86 73.66) (width 0.7) (layer F.Cu) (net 7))
 (segment (start 22.955 73.66) (end 25.55 76.255) (width 0.7) (layer F.Cu) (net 7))
 (segment (start 22.86 73.66) (end 22.955 73.66) (width 0.7) (layer F.Cu) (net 7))
 (segment (start 22.86 71.12) (end 22.86 68.58) (width 0.7) (layer F.Cu) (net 7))
 (segment (start 23.495 36.83) (end 27.94 41.275) (width 0.7) (layer F.Cu) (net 9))
 (segment (start 21.59 36.83) (end 23.495 36.83) (width 0.7) (layer F.Cu) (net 9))
 (segment (start 53.755 76.56) (end 58.835 76.56) (width 0.7) (layer F.Cu) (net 3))
 (segment (start 53.755 74.02) (end 58.835 74.02) (width 0.7) (layer F.Cu) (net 4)))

